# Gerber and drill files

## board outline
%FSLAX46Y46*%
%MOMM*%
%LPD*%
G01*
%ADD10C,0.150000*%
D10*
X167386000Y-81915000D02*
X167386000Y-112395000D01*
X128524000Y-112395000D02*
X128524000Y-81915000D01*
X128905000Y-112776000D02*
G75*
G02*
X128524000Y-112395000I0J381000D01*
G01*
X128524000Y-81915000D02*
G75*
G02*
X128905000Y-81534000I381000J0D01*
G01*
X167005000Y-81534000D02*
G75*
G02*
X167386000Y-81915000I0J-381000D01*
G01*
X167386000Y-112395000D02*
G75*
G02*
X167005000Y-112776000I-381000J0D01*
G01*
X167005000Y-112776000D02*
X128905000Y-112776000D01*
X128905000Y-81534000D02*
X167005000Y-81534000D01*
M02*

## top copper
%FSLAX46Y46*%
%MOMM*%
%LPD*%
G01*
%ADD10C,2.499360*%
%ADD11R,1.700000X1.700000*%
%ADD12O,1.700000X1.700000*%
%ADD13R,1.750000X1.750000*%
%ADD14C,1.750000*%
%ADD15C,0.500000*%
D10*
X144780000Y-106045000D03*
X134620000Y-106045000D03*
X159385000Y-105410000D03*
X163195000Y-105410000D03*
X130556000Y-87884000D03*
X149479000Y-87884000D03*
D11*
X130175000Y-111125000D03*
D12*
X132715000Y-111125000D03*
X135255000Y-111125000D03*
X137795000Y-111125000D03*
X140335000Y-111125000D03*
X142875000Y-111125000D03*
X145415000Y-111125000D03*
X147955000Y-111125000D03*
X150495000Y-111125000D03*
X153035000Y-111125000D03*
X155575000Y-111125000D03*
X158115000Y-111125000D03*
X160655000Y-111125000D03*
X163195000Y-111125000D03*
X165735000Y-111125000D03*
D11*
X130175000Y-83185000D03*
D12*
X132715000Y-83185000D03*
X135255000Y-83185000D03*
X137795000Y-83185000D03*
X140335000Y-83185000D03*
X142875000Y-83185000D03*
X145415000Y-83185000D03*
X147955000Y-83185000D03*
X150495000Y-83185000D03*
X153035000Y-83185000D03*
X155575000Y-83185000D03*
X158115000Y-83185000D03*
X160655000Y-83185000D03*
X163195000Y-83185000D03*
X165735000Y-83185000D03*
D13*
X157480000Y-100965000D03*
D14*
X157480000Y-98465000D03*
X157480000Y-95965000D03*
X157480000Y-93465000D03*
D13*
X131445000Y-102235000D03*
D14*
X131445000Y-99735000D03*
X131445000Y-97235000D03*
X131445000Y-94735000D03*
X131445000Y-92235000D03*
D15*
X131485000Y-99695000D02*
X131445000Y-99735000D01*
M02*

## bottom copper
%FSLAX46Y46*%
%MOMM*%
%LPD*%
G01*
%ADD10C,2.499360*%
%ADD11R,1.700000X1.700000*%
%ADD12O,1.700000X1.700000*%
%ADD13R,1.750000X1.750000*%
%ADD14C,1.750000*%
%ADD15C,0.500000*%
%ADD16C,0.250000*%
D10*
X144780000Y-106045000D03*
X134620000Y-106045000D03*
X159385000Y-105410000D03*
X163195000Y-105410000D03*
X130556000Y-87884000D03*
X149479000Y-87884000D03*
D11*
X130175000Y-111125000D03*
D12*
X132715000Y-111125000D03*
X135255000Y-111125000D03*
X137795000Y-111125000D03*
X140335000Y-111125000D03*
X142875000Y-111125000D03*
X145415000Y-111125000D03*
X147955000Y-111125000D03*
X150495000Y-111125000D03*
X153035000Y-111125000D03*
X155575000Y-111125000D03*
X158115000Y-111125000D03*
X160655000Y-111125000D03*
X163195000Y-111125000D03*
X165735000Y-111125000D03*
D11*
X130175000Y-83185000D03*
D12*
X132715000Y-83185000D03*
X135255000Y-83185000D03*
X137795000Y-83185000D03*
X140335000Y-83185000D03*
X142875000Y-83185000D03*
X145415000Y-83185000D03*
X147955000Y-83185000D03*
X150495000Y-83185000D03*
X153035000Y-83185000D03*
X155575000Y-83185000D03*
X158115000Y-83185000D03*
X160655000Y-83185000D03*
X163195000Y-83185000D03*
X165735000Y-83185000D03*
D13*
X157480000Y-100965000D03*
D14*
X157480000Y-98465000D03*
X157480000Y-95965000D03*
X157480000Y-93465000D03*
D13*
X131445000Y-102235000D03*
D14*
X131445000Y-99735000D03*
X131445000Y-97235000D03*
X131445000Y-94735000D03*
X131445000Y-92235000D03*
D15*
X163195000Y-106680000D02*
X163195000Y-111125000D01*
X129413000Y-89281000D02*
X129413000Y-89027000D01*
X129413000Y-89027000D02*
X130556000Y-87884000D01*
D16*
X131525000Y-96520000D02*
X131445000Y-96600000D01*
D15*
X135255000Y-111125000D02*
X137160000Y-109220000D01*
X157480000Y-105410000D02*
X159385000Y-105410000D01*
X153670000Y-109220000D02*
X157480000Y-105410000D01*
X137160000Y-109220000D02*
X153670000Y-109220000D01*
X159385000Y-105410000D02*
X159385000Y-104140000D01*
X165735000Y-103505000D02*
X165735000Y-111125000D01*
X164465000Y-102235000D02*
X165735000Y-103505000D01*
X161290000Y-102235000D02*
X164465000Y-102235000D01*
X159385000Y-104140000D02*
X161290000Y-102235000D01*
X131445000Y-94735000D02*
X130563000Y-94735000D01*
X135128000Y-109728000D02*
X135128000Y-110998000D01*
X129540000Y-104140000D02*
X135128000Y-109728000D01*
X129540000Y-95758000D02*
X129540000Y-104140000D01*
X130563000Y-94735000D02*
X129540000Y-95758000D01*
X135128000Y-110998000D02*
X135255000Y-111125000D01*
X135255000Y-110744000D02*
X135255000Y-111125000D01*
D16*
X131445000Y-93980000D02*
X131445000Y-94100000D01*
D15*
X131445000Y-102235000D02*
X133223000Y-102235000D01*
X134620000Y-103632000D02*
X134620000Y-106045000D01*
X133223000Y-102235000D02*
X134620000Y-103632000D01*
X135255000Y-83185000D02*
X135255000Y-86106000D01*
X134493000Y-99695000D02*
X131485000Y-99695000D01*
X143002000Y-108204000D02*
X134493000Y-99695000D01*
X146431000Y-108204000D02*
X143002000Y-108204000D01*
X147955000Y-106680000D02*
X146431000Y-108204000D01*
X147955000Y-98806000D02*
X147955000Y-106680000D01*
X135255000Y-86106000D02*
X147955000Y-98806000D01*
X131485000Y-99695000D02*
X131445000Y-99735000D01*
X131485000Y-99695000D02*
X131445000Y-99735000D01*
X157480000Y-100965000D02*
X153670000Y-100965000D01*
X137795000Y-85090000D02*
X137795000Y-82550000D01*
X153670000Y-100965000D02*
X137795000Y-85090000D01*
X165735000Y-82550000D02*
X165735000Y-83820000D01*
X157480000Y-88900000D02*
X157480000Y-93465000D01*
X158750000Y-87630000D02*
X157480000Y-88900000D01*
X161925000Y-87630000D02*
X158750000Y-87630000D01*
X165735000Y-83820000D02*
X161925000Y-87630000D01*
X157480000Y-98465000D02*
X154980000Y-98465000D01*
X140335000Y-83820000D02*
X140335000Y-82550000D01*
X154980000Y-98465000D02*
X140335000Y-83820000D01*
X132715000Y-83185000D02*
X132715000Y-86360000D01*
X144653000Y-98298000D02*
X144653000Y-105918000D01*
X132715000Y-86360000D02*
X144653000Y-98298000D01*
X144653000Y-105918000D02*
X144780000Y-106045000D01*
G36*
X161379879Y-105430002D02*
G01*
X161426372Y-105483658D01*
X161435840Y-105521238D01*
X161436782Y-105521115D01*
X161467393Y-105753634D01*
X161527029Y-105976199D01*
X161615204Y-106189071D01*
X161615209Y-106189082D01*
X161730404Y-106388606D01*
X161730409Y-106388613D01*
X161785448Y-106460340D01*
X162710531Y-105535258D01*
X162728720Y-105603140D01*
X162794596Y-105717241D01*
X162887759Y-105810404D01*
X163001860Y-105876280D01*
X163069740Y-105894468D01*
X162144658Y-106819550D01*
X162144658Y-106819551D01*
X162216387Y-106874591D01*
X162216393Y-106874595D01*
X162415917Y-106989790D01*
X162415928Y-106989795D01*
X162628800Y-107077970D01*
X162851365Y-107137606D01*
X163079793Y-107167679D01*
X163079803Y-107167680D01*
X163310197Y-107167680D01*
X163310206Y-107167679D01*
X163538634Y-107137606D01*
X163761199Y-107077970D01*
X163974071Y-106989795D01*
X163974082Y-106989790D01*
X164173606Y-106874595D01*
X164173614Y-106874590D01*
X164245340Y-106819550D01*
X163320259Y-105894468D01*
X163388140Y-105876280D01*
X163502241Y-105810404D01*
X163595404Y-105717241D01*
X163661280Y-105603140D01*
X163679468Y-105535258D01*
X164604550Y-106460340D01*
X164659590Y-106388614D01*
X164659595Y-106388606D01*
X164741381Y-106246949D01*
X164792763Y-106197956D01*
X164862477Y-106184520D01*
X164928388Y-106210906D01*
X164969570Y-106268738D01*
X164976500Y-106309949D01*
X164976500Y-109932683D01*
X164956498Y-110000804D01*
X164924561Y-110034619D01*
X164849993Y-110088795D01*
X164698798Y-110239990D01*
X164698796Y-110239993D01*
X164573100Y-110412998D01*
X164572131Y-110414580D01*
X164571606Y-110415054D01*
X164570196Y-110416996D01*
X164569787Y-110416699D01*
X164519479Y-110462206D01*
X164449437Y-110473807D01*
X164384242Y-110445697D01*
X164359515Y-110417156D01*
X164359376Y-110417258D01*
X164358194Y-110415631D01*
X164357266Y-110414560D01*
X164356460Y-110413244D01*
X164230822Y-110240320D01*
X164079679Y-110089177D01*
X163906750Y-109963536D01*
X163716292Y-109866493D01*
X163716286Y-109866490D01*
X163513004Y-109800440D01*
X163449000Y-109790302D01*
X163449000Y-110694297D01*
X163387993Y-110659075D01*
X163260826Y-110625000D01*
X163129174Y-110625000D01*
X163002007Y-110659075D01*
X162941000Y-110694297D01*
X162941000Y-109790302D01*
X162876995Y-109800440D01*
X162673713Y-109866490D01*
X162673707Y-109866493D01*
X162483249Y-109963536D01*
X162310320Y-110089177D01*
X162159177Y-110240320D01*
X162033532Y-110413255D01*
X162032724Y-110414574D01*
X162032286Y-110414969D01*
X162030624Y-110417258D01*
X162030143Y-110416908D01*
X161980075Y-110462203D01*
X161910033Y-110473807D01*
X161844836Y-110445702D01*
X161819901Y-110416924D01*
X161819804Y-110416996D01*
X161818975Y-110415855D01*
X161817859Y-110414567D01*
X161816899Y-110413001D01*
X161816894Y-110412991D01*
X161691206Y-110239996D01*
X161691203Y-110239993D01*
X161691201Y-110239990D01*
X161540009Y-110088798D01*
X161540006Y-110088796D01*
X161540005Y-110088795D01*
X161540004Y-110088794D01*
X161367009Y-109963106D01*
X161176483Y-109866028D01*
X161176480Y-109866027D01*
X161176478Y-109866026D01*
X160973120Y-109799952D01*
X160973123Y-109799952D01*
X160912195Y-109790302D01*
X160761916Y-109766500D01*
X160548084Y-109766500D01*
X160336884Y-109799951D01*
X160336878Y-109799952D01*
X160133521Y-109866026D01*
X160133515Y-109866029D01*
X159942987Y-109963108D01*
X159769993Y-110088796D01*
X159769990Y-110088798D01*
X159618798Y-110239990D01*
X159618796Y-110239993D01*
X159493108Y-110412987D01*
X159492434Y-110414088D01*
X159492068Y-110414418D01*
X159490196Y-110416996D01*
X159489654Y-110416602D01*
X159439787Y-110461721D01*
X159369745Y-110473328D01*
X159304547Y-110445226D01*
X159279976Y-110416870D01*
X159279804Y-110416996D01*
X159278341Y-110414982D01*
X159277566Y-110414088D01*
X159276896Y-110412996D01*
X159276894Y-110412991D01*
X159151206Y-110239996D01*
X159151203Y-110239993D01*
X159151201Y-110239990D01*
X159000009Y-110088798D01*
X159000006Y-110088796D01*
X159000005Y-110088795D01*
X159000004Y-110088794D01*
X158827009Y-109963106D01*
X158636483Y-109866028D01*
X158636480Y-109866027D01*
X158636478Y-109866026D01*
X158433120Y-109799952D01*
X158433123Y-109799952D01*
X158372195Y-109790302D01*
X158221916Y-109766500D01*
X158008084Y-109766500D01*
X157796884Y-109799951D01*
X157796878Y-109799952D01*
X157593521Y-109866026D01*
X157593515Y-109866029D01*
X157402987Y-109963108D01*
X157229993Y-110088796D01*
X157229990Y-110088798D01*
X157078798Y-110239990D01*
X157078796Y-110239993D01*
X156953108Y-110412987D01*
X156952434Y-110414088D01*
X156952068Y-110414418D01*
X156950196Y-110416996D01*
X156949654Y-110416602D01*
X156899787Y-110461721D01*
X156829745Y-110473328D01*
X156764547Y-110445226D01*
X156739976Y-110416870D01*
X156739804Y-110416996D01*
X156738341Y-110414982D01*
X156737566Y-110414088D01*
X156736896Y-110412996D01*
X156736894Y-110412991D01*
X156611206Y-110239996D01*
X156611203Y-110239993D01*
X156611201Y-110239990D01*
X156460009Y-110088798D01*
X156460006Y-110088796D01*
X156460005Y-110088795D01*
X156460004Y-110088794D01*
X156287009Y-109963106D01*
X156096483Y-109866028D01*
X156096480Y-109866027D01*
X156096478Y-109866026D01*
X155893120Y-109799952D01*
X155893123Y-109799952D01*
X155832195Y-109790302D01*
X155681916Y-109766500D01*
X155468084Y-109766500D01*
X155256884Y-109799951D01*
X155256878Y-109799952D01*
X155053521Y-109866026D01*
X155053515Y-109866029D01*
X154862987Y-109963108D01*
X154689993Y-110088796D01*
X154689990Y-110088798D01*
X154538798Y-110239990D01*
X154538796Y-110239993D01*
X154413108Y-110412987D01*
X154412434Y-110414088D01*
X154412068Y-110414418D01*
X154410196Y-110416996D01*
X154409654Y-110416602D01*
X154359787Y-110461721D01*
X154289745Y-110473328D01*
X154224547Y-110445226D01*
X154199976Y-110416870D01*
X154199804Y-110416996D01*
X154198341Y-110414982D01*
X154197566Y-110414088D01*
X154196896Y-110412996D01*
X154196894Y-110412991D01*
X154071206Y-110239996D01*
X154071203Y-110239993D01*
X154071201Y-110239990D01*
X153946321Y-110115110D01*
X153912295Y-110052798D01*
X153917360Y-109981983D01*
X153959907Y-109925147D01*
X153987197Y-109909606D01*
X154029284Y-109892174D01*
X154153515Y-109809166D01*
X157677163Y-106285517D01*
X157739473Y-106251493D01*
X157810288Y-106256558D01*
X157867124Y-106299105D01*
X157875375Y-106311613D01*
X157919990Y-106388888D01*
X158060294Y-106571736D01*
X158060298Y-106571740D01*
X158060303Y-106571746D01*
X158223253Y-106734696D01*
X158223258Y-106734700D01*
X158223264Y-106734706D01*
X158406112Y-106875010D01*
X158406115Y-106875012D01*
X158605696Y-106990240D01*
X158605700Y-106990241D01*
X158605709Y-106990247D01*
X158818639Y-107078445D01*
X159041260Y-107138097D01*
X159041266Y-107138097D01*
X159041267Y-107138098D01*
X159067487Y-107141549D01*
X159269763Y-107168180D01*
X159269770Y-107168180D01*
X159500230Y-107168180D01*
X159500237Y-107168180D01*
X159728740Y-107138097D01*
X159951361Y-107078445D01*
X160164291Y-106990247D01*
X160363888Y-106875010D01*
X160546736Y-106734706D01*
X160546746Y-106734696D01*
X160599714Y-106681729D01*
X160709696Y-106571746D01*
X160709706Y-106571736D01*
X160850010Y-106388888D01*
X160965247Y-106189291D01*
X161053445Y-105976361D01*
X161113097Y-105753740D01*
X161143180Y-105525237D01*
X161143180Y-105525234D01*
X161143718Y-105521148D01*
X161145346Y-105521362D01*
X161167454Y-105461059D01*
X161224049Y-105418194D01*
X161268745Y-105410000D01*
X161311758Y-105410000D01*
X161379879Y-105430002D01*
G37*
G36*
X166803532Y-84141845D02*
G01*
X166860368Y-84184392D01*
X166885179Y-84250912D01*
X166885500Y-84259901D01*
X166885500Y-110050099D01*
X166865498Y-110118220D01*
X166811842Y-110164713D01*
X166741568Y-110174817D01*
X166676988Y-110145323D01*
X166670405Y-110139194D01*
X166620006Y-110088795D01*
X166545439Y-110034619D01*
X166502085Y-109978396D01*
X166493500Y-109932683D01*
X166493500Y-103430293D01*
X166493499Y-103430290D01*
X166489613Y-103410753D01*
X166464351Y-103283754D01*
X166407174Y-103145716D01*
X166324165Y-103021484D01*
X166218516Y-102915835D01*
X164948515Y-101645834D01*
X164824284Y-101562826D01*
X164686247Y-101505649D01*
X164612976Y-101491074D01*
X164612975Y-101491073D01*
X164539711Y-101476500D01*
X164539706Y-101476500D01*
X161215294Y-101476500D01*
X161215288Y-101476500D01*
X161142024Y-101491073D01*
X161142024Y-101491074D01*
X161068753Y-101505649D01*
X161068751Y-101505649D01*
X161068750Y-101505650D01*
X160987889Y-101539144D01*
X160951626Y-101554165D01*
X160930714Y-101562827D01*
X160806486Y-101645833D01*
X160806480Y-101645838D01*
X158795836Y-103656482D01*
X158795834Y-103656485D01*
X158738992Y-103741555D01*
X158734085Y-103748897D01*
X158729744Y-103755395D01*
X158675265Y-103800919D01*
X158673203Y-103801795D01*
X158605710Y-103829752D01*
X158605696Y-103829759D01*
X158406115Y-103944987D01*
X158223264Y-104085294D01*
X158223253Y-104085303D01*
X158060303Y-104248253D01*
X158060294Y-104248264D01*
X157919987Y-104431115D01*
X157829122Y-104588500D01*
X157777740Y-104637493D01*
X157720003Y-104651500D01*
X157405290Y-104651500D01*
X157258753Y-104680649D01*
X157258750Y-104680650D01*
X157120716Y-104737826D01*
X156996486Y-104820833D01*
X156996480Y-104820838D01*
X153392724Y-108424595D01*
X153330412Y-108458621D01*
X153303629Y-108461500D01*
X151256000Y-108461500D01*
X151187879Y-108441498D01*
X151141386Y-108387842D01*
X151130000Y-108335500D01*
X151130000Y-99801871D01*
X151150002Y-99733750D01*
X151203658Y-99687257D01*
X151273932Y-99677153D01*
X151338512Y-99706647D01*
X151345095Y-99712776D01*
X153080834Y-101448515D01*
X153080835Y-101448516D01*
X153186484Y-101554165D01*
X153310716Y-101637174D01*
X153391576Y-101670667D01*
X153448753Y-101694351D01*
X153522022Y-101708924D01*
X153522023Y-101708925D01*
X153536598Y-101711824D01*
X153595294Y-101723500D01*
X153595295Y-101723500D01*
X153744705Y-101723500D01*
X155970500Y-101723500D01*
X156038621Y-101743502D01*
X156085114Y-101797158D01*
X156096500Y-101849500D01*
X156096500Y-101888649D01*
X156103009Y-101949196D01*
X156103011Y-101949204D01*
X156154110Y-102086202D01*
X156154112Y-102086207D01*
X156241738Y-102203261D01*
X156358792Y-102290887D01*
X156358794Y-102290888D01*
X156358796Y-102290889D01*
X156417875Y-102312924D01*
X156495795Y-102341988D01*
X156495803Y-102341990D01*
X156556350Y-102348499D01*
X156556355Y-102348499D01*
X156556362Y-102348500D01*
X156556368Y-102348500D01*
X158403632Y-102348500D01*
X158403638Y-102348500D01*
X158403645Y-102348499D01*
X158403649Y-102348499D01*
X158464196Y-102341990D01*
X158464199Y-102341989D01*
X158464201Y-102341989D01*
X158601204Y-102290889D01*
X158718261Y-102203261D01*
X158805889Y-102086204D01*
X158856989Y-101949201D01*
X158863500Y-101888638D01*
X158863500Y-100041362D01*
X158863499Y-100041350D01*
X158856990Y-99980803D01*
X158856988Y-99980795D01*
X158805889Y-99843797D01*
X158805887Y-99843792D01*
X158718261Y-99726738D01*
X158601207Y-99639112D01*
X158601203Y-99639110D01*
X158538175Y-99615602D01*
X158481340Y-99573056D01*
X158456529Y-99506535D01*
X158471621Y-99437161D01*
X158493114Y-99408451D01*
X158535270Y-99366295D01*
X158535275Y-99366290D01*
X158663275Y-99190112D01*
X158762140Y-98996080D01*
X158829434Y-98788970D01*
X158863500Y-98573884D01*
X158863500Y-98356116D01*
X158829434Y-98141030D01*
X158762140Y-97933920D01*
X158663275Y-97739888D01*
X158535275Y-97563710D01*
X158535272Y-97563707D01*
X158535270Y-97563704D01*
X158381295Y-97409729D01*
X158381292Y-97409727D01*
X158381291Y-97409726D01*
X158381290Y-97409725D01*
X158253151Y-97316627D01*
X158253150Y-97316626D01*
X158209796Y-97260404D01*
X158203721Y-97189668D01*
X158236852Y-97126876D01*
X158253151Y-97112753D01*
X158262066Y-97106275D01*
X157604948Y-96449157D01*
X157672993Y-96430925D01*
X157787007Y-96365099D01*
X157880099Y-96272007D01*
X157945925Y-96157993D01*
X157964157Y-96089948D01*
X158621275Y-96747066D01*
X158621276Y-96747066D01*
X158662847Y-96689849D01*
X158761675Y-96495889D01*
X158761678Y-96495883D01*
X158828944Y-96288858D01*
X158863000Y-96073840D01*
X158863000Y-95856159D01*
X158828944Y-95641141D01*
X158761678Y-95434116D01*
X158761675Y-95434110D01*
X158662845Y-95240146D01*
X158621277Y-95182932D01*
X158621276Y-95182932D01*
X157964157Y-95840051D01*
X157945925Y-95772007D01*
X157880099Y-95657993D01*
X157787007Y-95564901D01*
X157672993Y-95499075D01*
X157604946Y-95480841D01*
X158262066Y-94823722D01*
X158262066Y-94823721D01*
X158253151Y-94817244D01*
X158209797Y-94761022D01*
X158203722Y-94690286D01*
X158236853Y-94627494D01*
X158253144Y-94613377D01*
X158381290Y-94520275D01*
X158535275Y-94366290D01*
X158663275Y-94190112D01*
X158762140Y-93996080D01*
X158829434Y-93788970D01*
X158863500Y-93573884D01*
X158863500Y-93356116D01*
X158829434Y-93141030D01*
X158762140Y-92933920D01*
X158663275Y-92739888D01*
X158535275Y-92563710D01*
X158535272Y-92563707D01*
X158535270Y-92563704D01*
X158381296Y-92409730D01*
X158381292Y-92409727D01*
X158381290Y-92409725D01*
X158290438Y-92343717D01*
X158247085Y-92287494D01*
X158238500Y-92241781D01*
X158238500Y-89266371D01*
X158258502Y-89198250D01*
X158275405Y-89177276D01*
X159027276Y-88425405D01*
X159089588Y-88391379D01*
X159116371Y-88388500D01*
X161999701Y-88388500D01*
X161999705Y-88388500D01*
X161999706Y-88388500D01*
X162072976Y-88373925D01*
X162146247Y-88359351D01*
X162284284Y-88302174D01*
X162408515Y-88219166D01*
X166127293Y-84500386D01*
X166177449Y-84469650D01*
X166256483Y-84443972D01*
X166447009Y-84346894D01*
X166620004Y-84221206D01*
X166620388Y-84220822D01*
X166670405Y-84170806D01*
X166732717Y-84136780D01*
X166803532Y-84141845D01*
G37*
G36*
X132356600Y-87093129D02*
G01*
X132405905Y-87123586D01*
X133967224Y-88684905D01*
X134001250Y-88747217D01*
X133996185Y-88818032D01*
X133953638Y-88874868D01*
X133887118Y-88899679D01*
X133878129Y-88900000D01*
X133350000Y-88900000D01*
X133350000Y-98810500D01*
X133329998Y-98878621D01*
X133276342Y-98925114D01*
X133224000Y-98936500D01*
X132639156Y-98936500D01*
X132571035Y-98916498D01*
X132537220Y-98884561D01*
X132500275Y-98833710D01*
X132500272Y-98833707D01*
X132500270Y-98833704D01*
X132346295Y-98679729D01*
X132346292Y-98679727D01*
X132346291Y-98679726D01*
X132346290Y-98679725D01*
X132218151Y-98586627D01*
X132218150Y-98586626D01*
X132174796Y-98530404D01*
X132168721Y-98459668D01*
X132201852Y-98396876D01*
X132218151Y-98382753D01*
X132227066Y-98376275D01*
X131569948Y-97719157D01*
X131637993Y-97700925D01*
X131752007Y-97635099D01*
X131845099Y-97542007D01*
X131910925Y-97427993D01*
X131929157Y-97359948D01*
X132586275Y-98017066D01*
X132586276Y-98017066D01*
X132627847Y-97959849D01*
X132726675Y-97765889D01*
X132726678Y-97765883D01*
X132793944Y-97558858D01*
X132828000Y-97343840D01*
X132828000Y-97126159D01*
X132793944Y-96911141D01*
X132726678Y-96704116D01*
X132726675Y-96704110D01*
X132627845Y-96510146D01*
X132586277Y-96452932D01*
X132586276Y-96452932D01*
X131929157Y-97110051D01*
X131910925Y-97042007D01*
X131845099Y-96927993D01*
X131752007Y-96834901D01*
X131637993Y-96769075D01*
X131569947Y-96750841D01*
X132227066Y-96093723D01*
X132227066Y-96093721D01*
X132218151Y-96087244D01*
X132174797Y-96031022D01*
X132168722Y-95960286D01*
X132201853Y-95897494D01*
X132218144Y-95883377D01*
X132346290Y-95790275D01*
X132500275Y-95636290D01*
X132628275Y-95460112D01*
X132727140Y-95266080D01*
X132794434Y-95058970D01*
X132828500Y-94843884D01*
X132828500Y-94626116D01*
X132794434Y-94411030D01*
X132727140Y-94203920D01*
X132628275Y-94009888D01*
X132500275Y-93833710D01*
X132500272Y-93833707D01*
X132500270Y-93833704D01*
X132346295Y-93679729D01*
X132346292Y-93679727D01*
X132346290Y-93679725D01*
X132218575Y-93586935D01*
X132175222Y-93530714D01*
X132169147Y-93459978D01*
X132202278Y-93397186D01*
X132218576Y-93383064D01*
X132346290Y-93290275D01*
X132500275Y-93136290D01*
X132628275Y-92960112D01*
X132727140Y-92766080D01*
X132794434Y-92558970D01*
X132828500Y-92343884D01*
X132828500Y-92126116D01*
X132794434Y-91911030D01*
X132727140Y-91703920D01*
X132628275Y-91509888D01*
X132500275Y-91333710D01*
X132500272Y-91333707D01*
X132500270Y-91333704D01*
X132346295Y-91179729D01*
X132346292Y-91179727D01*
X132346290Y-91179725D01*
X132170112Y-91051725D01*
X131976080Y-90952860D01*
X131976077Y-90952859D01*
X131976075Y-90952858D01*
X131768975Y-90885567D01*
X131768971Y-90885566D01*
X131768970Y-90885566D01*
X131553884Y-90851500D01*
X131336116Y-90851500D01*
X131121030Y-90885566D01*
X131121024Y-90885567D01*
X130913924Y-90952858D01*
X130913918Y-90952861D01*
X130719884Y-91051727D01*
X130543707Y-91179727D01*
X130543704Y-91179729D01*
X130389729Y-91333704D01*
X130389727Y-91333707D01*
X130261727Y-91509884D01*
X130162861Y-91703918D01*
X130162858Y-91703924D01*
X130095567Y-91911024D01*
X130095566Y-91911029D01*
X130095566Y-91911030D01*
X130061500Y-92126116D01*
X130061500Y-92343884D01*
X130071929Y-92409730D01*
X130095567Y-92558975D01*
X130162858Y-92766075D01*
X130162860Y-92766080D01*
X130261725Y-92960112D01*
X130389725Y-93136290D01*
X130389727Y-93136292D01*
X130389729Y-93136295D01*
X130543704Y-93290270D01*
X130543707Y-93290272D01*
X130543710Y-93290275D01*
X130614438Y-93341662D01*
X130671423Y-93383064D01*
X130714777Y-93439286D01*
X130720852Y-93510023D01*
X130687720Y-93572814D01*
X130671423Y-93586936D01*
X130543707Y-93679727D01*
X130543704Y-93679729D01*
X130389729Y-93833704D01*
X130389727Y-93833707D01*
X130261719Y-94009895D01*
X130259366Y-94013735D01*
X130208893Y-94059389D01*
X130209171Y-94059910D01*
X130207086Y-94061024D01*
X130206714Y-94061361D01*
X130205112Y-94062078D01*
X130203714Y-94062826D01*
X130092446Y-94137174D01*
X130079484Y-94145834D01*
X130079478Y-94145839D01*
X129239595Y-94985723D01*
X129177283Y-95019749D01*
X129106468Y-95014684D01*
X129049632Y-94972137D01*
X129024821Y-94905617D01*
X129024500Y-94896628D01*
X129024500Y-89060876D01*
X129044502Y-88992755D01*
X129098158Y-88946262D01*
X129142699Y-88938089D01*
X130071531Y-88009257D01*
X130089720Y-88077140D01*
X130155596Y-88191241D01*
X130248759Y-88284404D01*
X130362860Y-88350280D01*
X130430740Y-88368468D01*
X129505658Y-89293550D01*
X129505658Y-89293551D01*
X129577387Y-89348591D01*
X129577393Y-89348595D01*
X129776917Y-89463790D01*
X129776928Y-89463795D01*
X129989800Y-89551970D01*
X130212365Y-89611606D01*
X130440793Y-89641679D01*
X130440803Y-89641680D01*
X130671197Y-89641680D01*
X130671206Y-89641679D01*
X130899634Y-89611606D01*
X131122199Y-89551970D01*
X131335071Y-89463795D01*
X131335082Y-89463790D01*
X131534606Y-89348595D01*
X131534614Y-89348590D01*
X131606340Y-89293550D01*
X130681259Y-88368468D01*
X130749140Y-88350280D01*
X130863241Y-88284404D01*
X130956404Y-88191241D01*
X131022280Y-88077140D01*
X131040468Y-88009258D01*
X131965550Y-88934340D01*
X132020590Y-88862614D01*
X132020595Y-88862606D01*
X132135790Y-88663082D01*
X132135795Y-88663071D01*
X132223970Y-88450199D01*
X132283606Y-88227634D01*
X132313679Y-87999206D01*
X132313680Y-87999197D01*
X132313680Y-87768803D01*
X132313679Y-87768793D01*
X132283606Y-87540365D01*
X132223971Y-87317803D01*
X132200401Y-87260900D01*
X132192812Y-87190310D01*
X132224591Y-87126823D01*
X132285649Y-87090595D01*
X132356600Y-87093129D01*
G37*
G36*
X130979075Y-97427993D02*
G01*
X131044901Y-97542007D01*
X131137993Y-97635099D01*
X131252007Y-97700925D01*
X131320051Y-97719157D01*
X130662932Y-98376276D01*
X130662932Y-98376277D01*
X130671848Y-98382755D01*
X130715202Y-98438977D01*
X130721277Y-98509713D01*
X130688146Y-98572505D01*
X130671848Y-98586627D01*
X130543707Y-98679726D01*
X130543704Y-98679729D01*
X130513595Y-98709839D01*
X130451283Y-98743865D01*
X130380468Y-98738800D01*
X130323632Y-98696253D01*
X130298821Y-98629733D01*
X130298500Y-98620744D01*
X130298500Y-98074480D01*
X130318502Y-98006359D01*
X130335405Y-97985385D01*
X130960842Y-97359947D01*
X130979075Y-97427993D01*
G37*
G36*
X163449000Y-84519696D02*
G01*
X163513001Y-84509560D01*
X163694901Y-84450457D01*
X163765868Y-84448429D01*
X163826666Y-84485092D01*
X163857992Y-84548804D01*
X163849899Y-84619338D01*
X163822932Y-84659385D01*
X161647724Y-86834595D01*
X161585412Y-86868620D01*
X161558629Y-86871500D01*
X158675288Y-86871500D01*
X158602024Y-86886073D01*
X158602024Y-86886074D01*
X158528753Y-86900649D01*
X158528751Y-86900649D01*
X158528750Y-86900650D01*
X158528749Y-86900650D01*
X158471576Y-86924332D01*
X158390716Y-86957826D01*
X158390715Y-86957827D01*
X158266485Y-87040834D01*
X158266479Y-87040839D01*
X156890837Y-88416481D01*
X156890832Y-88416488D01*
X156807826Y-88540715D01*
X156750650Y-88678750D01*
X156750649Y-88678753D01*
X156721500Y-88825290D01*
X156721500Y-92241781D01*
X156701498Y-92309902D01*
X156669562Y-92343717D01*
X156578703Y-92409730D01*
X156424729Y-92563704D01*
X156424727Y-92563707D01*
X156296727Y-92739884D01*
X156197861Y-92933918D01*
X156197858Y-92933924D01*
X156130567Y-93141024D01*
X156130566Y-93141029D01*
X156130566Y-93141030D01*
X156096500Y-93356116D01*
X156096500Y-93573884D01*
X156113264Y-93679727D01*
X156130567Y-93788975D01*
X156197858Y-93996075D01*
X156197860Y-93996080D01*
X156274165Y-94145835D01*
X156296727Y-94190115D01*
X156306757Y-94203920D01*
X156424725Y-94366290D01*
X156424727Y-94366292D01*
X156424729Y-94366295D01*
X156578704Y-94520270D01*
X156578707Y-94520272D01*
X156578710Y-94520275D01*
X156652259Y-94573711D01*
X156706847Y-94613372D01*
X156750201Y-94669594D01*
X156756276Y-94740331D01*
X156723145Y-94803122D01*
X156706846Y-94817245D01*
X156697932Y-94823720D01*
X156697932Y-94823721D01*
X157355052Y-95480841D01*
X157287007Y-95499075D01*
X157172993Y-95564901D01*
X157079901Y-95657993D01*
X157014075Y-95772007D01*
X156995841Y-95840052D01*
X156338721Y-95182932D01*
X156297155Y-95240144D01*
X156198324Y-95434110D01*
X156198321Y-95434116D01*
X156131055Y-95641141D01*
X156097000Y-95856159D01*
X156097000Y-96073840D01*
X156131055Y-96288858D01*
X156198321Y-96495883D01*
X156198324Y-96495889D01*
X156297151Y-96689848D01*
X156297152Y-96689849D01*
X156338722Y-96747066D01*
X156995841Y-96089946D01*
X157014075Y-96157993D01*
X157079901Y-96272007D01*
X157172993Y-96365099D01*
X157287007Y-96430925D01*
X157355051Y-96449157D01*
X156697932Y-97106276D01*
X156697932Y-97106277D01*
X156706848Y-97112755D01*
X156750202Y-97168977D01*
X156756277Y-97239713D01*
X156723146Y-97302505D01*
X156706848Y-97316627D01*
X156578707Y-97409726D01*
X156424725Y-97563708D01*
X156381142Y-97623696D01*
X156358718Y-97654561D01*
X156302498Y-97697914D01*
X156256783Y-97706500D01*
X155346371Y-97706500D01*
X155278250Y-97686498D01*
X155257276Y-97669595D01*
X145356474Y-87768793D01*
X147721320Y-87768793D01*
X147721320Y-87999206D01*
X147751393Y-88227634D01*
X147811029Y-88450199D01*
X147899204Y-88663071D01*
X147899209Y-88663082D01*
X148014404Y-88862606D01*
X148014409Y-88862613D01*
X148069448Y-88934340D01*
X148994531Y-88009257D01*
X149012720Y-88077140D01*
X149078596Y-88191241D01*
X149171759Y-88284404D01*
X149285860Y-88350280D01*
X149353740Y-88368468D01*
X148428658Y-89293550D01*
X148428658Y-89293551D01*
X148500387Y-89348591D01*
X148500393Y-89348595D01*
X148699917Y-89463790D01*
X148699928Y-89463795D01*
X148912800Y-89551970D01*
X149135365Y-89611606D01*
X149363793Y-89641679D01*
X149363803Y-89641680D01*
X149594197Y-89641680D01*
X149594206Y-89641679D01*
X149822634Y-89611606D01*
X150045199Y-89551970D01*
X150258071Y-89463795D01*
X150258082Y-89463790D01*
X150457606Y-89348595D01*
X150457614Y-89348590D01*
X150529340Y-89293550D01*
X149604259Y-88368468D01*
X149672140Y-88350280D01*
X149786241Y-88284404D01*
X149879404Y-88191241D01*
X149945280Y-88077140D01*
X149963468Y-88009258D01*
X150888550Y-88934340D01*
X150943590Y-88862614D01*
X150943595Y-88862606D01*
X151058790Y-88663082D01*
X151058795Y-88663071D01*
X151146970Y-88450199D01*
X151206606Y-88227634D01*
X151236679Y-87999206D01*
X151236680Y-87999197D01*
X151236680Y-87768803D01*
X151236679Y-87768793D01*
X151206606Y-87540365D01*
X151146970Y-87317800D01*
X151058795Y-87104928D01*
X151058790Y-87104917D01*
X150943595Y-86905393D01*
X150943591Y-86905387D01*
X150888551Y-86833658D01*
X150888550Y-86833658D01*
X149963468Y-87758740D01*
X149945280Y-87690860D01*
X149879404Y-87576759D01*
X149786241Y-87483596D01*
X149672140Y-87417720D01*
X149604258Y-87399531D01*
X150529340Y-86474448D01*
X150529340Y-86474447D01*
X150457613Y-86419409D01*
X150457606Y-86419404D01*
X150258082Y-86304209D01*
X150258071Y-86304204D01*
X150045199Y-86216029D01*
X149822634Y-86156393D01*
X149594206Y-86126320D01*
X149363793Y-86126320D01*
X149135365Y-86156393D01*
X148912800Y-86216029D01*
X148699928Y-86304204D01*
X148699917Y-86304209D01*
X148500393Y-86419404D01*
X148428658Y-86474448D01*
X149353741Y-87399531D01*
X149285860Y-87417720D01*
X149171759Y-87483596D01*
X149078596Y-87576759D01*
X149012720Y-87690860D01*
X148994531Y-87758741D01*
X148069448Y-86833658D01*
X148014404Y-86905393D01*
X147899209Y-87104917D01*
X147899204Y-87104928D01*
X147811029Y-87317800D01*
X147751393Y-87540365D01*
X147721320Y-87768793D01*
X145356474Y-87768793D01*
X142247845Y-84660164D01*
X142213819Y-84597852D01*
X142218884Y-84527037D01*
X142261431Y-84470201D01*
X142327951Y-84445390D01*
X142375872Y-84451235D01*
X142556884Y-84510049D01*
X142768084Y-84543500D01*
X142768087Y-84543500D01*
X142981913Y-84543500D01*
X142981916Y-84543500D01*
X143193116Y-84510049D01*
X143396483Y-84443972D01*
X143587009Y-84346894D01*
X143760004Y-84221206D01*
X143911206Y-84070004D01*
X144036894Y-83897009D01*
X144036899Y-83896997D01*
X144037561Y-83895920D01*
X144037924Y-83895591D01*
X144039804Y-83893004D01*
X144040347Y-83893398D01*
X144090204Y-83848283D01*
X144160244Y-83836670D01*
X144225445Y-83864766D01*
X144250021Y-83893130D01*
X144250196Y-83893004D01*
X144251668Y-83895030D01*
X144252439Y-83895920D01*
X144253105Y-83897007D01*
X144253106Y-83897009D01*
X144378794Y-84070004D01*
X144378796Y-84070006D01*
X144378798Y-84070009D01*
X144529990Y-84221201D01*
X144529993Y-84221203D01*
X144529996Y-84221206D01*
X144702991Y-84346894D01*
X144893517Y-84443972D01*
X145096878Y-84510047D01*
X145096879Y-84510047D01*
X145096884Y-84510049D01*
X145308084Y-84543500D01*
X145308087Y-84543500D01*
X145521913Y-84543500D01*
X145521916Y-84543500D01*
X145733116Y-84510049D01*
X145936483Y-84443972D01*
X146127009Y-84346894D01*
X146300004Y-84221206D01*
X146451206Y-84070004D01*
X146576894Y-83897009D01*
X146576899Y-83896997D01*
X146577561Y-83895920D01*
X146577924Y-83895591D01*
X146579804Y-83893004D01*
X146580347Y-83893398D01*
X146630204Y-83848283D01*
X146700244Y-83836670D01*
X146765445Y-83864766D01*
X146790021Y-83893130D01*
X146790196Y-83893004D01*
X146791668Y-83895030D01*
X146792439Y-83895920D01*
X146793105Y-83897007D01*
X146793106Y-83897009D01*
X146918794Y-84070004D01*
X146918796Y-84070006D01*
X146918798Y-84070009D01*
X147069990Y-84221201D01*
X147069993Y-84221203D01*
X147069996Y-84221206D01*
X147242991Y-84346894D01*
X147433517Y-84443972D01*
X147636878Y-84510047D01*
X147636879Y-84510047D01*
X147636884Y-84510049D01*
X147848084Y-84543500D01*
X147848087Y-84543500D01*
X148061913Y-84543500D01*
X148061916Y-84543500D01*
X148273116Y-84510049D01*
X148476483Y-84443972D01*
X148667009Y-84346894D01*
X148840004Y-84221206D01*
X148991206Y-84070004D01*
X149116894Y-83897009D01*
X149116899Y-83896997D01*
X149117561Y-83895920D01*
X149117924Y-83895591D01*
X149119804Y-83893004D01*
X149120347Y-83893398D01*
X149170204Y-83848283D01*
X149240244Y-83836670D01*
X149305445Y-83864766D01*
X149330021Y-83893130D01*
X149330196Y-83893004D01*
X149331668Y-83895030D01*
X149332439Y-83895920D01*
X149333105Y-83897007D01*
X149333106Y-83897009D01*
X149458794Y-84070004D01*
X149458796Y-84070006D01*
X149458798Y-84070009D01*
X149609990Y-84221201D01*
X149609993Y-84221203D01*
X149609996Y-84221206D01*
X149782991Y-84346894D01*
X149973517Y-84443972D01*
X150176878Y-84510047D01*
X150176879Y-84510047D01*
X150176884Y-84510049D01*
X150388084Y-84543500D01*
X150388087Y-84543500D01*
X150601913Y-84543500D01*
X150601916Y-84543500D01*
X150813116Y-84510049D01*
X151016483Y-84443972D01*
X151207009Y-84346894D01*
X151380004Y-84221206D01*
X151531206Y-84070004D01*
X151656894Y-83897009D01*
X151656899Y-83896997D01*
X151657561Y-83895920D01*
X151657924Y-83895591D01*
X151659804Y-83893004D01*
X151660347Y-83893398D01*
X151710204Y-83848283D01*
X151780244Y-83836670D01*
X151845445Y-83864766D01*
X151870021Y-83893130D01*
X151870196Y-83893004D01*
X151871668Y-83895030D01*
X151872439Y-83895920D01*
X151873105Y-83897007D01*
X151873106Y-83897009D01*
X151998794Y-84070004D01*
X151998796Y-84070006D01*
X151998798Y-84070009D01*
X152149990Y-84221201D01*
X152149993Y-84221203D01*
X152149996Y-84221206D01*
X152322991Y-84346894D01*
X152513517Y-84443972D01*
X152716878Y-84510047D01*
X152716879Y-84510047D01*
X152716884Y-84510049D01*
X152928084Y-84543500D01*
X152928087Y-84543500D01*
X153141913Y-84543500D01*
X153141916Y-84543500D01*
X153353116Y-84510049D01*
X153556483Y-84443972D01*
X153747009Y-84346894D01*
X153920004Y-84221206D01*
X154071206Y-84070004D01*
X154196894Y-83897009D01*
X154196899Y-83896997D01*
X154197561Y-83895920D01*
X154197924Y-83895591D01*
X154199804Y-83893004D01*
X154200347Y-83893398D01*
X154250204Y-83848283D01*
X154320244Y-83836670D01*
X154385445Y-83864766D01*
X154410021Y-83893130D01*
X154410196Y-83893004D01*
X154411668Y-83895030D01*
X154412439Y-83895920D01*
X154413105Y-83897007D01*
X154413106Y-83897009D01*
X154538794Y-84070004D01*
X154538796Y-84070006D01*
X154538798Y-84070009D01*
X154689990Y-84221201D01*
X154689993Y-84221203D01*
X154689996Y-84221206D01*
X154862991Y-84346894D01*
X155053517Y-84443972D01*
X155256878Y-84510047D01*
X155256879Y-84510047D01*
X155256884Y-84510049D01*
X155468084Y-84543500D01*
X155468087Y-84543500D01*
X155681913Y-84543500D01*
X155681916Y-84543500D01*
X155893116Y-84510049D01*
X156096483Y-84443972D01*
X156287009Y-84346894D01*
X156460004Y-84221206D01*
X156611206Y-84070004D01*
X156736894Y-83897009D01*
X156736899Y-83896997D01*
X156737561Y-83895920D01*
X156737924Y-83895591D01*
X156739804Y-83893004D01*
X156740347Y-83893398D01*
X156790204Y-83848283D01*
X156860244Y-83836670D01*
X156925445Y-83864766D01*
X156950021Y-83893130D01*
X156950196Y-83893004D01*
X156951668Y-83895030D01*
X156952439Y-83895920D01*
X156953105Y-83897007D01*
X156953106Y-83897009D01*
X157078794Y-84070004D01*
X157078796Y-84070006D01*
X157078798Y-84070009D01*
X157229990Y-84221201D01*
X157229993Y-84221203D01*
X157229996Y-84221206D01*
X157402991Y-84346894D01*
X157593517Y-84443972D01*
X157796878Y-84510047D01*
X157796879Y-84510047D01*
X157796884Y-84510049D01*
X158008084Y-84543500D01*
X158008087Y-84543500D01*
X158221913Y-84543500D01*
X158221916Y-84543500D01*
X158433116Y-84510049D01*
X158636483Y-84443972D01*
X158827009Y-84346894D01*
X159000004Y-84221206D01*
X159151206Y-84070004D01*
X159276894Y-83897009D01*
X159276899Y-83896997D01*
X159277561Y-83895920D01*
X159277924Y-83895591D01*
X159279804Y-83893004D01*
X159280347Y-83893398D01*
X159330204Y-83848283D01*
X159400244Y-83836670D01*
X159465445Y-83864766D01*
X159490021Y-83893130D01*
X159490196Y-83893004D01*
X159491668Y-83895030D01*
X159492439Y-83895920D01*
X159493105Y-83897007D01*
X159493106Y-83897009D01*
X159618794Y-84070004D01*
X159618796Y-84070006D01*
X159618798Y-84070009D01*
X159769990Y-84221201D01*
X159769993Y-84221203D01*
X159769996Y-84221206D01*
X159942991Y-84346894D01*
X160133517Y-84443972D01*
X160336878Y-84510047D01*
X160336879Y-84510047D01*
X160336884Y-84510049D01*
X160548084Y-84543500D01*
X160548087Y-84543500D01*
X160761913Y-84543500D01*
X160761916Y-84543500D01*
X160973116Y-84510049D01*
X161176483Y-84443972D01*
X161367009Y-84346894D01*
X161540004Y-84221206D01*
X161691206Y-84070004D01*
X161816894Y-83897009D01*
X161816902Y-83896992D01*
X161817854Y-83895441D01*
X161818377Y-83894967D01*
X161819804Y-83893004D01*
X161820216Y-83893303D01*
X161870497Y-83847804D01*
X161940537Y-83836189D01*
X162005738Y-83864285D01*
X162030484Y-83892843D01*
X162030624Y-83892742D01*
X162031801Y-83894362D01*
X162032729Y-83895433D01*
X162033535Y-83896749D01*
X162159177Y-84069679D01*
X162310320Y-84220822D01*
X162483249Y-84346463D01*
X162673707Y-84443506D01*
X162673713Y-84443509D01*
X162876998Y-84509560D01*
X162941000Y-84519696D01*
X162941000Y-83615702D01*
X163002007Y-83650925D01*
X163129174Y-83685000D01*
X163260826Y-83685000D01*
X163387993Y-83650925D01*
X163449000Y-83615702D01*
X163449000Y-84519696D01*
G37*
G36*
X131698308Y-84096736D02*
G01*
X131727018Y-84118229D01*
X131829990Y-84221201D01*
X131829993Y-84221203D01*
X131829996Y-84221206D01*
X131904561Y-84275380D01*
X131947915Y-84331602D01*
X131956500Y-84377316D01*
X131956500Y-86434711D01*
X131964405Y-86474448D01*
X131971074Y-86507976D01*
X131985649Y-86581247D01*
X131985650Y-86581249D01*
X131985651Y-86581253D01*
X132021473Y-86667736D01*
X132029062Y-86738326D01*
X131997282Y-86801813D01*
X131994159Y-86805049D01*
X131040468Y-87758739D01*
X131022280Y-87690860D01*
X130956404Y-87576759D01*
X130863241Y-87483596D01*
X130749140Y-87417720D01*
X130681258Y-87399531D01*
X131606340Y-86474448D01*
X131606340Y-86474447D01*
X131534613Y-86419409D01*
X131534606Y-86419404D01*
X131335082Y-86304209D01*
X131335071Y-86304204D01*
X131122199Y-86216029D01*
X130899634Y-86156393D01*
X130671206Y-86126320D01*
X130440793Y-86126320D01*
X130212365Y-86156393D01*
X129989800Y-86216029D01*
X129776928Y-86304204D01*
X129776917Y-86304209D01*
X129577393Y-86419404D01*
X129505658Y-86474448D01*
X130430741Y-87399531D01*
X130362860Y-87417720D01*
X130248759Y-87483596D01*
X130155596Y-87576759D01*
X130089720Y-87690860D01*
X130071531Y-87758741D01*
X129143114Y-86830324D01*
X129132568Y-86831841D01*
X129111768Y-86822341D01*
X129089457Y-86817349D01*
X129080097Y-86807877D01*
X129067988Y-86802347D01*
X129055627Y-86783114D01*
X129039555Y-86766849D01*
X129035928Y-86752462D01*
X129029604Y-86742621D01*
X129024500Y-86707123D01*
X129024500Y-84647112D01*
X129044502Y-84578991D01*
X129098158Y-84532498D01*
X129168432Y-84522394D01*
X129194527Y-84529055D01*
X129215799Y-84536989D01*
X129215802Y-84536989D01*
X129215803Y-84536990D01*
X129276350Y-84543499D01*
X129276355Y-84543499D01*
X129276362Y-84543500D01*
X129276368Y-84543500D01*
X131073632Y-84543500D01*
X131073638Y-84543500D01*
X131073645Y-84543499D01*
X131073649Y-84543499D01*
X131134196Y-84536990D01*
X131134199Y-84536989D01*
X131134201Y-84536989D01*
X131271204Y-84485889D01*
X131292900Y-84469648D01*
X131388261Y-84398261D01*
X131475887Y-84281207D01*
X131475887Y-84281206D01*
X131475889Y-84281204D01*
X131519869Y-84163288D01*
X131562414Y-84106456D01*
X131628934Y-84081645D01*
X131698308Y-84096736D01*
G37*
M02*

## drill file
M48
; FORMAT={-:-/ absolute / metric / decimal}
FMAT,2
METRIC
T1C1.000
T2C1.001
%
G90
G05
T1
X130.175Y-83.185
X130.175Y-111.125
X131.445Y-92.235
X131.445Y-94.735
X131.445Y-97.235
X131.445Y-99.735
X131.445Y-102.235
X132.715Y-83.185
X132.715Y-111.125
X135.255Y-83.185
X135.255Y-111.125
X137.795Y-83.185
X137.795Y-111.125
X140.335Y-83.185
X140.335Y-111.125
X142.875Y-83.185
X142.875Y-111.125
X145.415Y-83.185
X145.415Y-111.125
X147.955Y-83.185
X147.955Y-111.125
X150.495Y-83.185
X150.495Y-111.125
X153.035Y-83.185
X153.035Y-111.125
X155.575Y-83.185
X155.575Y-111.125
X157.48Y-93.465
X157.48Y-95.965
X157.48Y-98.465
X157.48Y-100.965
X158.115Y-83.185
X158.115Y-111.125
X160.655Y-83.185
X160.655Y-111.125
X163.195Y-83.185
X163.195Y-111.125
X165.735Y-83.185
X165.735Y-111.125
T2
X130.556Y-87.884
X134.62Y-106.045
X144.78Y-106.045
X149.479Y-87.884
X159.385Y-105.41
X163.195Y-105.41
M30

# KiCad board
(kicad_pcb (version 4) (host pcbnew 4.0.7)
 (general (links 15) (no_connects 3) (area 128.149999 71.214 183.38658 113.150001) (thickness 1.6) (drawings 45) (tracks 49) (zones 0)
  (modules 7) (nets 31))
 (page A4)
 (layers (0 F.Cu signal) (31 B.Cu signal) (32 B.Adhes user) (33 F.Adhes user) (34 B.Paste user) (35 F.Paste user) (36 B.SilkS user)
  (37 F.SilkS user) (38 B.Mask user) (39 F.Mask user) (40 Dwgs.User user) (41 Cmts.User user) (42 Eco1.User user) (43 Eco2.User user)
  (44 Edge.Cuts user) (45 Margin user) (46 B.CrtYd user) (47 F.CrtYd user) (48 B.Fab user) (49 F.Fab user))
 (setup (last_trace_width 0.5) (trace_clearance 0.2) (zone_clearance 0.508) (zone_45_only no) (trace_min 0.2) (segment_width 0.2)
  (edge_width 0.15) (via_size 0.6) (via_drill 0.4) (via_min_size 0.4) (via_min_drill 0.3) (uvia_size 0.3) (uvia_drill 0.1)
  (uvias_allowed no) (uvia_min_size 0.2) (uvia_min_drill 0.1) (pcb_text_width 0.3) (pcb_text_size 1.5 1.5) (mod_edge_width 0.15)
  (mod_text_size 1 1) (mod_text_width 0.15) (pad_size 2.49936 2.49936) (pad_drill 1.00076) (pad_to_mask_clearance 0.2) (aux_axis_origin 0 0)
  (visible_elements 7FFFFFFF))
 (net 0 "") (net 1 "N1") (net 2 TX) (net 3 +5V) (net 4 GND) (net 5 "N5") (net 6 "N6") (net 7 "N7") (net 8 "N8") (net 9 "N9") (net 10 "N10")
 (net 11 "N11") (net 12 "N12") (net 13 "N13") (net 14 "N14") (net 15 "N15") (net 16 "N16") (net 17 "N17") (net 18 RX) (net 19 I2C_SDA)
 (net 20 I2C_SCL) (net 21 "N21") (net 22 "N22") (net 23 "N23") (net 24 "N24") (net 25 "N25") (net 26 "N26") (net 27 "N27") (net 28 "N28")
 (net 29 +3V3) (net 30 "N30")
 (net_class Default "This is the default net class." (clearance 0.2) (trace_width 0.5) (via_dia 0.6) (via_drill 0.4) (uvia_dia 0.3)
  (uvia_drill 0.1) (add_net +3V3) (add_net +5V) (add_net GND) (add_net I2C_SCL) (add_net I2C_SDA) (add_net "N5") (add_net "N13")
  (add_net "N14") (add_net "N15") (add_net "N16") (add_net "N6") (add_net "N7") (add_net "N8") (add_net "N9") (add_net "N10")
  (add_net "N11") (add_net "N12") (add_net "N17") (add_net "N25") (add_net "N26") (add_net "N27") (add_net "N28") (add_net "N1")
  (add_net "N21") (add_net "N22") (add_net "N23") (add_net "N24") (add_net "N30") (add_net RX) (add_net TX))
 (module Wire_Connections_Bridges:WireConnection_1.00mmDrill (layer F.Cu) (at 144.78 106.045 180)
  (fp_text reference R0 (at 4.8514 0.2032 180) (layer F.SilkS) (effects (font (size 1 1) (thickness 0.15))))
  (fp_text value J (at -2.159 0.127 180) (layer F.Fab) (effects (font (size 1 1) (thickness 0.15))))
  (pad 1 thru_hole circle (at 0 0 180) (size 2.49936 2.49936) (drill 1.00076) (layers *.Cu *.Mask) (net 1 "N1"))
  (pad 2 thru_hole circle (at 10.16 0 180) (size 2.49936 2.49936) (drill 1.00076) (layers *.Cu *.Mask) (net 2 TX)))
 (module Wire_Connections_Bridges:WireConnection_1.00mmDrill (layer F.Cu) (at 156.845 105.41)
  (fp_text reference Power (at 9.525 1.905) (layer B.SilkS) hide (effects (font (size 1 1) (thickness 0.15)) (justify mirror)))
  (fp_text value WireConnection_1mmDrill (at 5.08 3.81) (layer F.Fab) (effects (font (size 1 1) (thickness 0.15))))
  (pad 1 thru_hole circle (at 2.54 0) (size 2.49936 2.49936) (drill 1.00076) (layers *.Cu *.Mask) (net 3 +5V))
  (pad 2 thru_hole circle (at 6.35 0) (size 2.49936 2.49936) (drill 1.00076) (layers *.Cu *.Mask) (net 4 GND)))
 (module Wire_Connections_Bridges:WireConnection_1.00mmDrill (layer F.Cu) (at 130.556 88.011)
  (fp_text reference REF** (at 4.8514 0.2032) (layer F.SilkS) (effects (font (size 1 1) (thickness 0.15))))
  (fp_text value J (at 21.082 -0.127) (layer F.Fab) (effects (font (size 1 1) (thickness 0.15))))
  (pad 1 thru_hole circle (at 0 -0.127) (size 2.49936 2.49936) (drill 1.00076) (layers *.Cu *.Mask) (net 4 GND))
  (pad 2 thru_hole circle (at 18.923 -0.127) (size 2.49936 2.49936) (drill 1.00076) (layers *.Cu *.Mask) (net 4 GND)))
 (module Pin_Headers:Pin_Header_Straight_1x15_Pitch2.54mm (layer F.Cu) (at 130.175 111.125 90)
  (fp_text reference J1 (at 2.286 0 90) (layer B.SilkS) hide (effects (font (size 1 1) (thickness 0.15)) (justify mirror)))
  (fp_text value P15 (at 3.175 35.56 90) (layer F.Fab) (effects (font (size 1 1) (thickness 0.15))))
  (pad 1 thru_hole rect (at 0 0 90) (size 1.7 1.7) (drill 1) (layers *.Cu *.Mask) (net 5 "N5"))
  (pad 2 thru_hole oval (at 0 2.54 90) (size 1.7 1.7) (drill 1) (layers *.Cu *.Mask) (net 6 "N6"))
  (pad 3 thru_hole oval (at 0 5.08 90) (size 1.7 1.7) (drill 1) (layers *.Cu *.Mask) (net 3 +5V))
  (pad 4 thru_hole oval (at 0 7.62 90) (size 1.7 1.7) (drill 1) (layers *.Cu *.Mask) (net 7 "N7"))
  (pad 5 thru_hole oval (at 0 10.16 90) (size 1.7 1.7) (drill 1) (layers *.Cu *.Mask) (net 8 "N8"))
  (pad 6 thru_hole oval (at 0 12.7 90) (size 1.7 1.7) (drill 1) (layers *.Cu *.Mask) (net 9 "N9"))
  (pad 7 thru_hole oval (at 0 15.24 90) (size 1.7 1.7) (drill 1) (layers *.Cu *.Mask) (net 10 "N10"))
  (pad 8 thru_hole oval (at 0 17.78 90) (size 1.7 1.7) (drill 1) (layers *.Cu *.Mask) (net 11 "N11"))
  (pad 9 thru_hole oval (at 0 20.32 90) (size 1.7 1.7) (drill 1) (layers *.Cu *.Mask) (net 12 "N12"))
  (pad 10 thru_hole oval (at 0 22.86 90) (size 1.7 1.7) (drill 1) (layers *.Cu *.Mask) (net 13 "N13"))
  (pad 11 thru_hole oval (at 0 25.4 90) (size 1.7 1.7) (drill 1) (layers *.Cu *.Mask) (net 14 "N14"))
  (pad 12 thru_hole oval (at 0 27.94 90) (size 1.7 1.7) (drill 1) (layers *.Cu *.Mask) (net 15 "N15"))
  (pad 13 thru_hole oval (at 0 30.48 90) (size 1.7 1.7) (drill 1) (layers *.Cu *.Mask) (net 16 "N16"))
  (pad 14 thru_hole oval (at 0 33.02 90) (size 1.7 1.7) (drill 1) (layers *.Cu *.Mask) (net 4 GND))
  (pad 15 thru_hole oval (at 0 35.56 90) (size 1.7 1.7) (drill 1) (layers *.Cu *.Mask) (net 3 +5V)))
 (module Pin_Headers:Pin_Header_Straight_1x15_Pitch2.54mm (layer F.Cu) (at 130.175 83.185 90)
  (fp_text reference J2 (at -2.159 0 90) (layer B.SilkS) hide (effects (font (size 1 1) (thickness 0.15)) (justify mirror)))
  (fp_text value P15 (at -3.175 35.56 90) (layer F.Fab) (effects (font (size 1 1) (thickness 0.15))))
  (pad 1 thru_hole rect (at 0 0 90) (size 1.7 1.7) (drill 1) (layers *.Cu *.Mask) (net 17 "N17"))
  (pad 2 thru_hole oval (at 0 2.54 90) (size 1.7 1.7) (drill 1) (layers *.Cu *.Mask) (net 1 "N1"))
  (pad 3 thru_hole oval (at 0 5.08 90) (size 1.7 1.7) (drill 1) (layers *.Cu *.Mask) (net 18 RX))
  (pad 4 thru_hole oval (at 0 7.62 90) (size 1.7 1.7) (drill 1) (layers *.Cu *.Mask) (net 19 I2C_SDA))
  (pad 5 thru_hole oval (at 0 10.16 90) (size 1.7 1.7) (drill 1) (layers *.Cu *.Mask) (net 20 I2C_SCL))
  (pad 6 thru_hole oval (at 0 12.7 90) (size 1.7 1.7) (drill 1) (layers *.Cu *.Mask) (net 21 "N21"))
  (pad 7 thru_hole oval (at 0 15.24 90) (size 1.7 1.7) (drill 1) (layers *.Cu *.Mask) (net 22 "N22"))
  (pad 8 thru_hole oval (at 0 17.78 90) (size 1.7 1.7) (drill 1) (layers *.Cu *.Mask) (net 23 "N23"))
  (pad 9 thru_hole oval (at 0 20.32 90) (size 1.7 1.7) (drill 1) (layers *.Cu *.Mask) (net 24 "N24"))
  (pad 10 thru_hole oval (at 0 22.86 90) (size 1.7 1.7) (drill 1) (layers *.Cu *.Mask) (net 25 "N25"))
  (pad 11 thru_hole oval (at 0 25.4 90) (size 1.7 1.7) (drill 1) (layers *.Cu *.Mask) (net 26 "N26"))
  (pad 12 thru_hole oval (at 0 27.94 90) (size 1.7 1.7) (drill 1) (layers *.Cu *.Mask) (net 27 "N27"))
  (pad 13 thru_hole oval (at 0 30.48 90) (size 1.7 1.7) (drill 1) (layers *.Cu *.Mask) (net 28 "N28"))
  (pad 14 thru_hole oval (at 0 33.02 90) (size 1.7 1.7) (drill 1) (layers *.Cu *.Mask) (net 4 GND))
  (pad 15 thru_hole oval (at 0 35.56 90) (size 1.7 1.7) (drill 1) (layers *.Cu *.Mask) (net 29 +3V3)))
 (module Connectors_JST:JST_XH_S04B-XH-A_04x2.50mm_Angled (layer F.Cu) (at 157.48 100.965 90)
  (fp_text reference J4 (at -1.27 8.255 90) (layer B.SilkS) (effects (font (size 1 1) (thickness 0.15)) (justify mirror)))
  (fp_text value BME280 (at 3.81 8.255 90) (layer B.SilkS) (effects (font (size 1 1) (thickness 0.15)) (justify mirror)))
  (pad 1 thru_hole rect (at 0 0 90) (size 1.75 1.75) (drill 1) (layers *.Cu *.Mask F.SilkS) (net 19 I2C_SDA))
  (pad 2 thru_hole circle (at 2.5 0 90) (size 1.75 1.75) (drill 1) (layers *.Cu *.Mask F.SilkS) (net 20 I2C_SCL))
  (pad 3 thru_hole circle (at 5 0 90) (size 1.75 1.75) (drill 1) (layers *.Cu *.Mask F.SilkS) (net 4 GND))
  (pad 4 thru_hole circle (at 7.5 0 90) (size 1.75 1.75) (drill 1) (layers *.Cu *.Mask F.SilkS) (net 29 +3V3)))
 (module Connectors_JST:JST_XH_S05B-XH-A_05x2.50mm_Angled (layer F.Cu) (at 131.445 102.235 90)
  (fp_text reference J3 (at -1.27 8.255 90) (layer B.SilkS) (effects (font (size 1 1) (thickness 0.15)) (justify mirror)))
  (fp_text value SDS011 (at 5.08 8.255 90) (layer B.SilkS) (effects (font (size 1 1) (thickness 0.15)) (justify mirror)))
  (pad 1 thru_hole rect (at 0 0 90) (size 1.75 1.75) (drill 1) (layers *.Cu *.Mask F.SilkS) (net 2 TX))
  (pad 2 thru_hole circle (at 2.5 0 90) (size 1.75 1.75) (drill 1) (layers *.Cu *.Mask F.SilkS) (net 18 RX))
  (pad 3 thru_hole circle (at 5 0 90) (size 1.75 1.75) (drill 1) (layers *.Cu *.Mask F.SilkS) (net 4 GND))
  (pad 4 thru_hole circle (at 7.5 0 90) (size 1.75 1.75) (drill 1) (layers *.Cu *.Mask F.SilkS) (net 3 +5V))
  (pad 5 thru_hole circle (at 10 0 90) (size 1.75 1.75) (drill 1) (layers *.Cu *.Mask F.SilkS) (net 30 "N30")))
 (gr_line (start 167.386 81.915) (end 167.386 112.395) (angle 90) (layer Edge.Cuts) (width 0.15))
 (gr_line (start 128.524 112.395) (end 128.524 81.915) (angle 90) (layer Edge.Cuts) (width 0.15))
 (gr_arc (start 128.905 112.395) (end 128.905 112.776) (angle 90) (layer Edge.Cuts) (width 0.15))
 (gr_arc (start 128.905 81.915) (end 128.524 81.915) (angle 90) (layer Edge.Cuts) (width 0.15))
 (gr_arc (start 167.005 81.915) (end 167.005 81.534) (angle 90) (layer Edge.Cuts) (width 0.15))
 (gr_arc (start 167.005 112.395) (end 167.386 112.395) (angle 90) (layer Edge.Cuts) (width 0.15))
 (gr_line (start 167.005 112.776) (end 128.905 112.776) (angle 90) (layer Edge.Cuts) (width 0.15))
 (gr_line (start 128.905 81.534) (end 167.005 81.534) (angle 90) (layer Edge.Cuts) (width 0.15))
 (segment (start 163.195 106.68) (end 163.195 111.125) (width 0.5) (layer B.Cu) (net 4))
 (segment (start 129.413 89.281) (end 129.413 89.027) (width 0.5) (layer B.Cu) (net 4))
 (segment (start 129.413 89.027) (end 130.556 87.884) (width 0.5) (layer B.Cu) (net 4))
 (segment (start 131.525 96.52) (end 131.445 96.6) (width 0.25) (layer B.Cu) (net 4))
 (segment (start 135.255 111.125) (end 137.16 109.22) (width 0.5) (layer B.Cu) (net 3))
 (segment (start 157.48 105.41) (end 159.385 105.41) (width 0.5) (layer B.Cu) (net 3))
 (segment (start 153.67 109.22) (end 157.48 105.41) (width 0.5) (layer B.Cu) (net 3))
 (segment (start 137.16 109.22) (end 153.67 109.22) (width 0.5) (layer B.Cu) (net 3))
 (segment (start 159.385 105.41) (end 159.385 104.14) (width 0.5) (layer B.Cu) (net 3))
 (segment (start 165.735 103.505) (end 165.735 111.125) (width 0.5) (layer B.Cu) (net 3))
 (segment (start 164.465 102.235) (end 165.735 103.505) (width 0.5) (layer B.Cu) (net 3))
 (segment (start 161.29 102.235) (end 164.465 102.235) (width 0.5) (layer B.Cu) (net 3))
 (segment (start 159.385 104.14) (end 161.29 102.235) (width 0.5) (layer B.Cu) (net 3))
 (segment (start 131.445 94.735) (end 130.563 94.735) (width 0.5) (layer B.Cu) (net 3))
 (segment (start 135.128 109.728) (end 135.128 110.998) (width 0.5) (layer B.Cu) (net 3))
 (segment (start 129.54 104.14) (end 135.128 109.728) (width 0.5) (layer B.Cu) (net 3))
 (segment (start 129.54 95.758) (end 129.54 104.14) (width 0.5) (layer B.Cu) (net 3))
 (segment (start 130.563 94.735) (end 129.54 95.758) (width 0.5) (layer B.Cu) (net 3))
 (segment (start 135.128 110.998) (end 135.255 111.125) (width 0.5) (layer B.Cu) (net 3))
 (segment (start 135.255 110.744) (end 135.255 111.125) (width 0.5) (layer B.Cu) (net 3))
 (segment (start 131.445 93.98) (end 131.445 94.1) (width 0.25) (layer B.Cu) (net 3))
 (segment (start 131.445 102.235) (end 133.223 102.235) (width 0.5) (layer B.Cu) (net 2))
 (segment (start 134.62 103.632) (end 134.62 106.045) (width 0.5) (layer B.Cu) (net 2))
 (segment (start 133.223 102.235) (end 134.62 103.632) (width 0.5) (layer B.Cu) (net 2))
 (segment (start 135.255 83.185) (end 135.255 86.106) (width 0.5) (layer B.Cu) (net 18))
 (segment (start 134.493 99.695) (end 131.485 99.695) (width 0.5) (layer B.Cu) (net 18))
 (segment (start 143.002 108.204) (end 134.493 99.695) (width 0.5) (layer B.Cu) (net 18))
 (segment (start 146.431 108.204) (end 143.002 108.204) (width 0.5) (layer B.Cu) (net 18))
 (segment (start 147.955 106.68) (end 146.431 108.204) (width 0.5) (layer B.Cu) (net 18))
 (segment (start 147.955 98.806) (end 147.955 106.68) (width 0.5) (layer B.Cu) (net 18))
 (segment (start 135.255 86.106) (end 147.955 98.806) (width 0.5) (layer B.Cu) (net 18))
 (segment (start 131.485 99.695) (end 131.445 99.735) (width 0.5) (layer B.Cu) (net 18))
 (segment (start 131.485 99.695) (end 131.445 99.735) (width 0.5) (layer F.Cu) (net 18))
 (segment (start 131.485 99.695) (end 131.445 99.735) (width 0.5) (layer B.Cu) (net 18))
 (segment (start 157.48 100.965) (end 153.67 100.965) (width 0.5) (layer B.Cu) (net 19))
 (segment (start 137.795 85.09) (end 137.795 82.55) (width 0.5) (layer B.Cu) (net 19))
 (segment (start 153.67 100.965) (end 137.795 85.09) (width 0.5) (layer B.Cu) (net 19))
 (segment (start 165.735 82.55) (end 165.735 83.82) (width 0.5) (layer B.Cu) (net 29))
 (segment (start 157.48 88.9) (end 157.48 93.465) (width 0.5) (layer B.Cu) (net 29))
 (segment (start 158.75 87.63) (end 157.48 88.9) (width 0.5) (layer B.Cu) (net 29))
 (segment (start 161.925 87.63) (end 158.75 87.63) (width 0.5) (layer B.Cu) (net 29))
 (segment (start 165.735 83.82) (end 161.925 87.63) (width 0.5) (layer B.Cu) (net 29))
 (segment (start 157.48 98.465) (end 154.98 98.465) (width 0.5) (layer B.Cu) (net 20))
 (segment (start 140.335 83.82) (end 140.335 82.55) (width 0.5) (layer B.Cu) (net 20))
 (segment (start 154.98 98.465) (end 140.335 83.82) (width 0.5) (layer B.Cu) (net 20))
 (segment (start 132.715 83.185) (end 132.715 86.36) (width 0.5) (layer B.Cu) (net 1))
 (segment (start 144.653 98.298) (end 144.653 105.918) (width 0.5) (layer B.Cu) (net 1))
 (segment (start 132.715 86.36) (end 144.653 98.298) (width 0.5) (layer B.Cu) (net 1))
 (segment (start 144.653 105.918) (end 144.78 106.045) (width 0.5) (layer B.Cu) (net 1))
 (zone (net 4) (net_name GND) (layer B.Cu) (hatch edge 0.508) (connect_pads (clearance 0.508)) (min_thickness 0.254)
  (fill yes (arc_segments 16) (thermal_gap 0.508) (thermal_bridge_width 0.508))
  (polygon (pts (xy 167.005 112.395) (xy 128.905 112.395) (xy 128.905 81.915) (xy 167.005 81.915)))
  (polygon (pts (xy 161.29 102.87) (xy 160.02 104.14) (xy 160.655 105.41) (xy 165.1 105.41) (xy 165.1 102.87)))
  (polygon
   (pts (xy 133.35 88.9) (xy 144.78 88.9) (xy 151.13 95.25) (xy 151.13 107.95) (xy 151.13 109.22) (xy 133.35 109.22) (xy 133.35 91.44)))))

